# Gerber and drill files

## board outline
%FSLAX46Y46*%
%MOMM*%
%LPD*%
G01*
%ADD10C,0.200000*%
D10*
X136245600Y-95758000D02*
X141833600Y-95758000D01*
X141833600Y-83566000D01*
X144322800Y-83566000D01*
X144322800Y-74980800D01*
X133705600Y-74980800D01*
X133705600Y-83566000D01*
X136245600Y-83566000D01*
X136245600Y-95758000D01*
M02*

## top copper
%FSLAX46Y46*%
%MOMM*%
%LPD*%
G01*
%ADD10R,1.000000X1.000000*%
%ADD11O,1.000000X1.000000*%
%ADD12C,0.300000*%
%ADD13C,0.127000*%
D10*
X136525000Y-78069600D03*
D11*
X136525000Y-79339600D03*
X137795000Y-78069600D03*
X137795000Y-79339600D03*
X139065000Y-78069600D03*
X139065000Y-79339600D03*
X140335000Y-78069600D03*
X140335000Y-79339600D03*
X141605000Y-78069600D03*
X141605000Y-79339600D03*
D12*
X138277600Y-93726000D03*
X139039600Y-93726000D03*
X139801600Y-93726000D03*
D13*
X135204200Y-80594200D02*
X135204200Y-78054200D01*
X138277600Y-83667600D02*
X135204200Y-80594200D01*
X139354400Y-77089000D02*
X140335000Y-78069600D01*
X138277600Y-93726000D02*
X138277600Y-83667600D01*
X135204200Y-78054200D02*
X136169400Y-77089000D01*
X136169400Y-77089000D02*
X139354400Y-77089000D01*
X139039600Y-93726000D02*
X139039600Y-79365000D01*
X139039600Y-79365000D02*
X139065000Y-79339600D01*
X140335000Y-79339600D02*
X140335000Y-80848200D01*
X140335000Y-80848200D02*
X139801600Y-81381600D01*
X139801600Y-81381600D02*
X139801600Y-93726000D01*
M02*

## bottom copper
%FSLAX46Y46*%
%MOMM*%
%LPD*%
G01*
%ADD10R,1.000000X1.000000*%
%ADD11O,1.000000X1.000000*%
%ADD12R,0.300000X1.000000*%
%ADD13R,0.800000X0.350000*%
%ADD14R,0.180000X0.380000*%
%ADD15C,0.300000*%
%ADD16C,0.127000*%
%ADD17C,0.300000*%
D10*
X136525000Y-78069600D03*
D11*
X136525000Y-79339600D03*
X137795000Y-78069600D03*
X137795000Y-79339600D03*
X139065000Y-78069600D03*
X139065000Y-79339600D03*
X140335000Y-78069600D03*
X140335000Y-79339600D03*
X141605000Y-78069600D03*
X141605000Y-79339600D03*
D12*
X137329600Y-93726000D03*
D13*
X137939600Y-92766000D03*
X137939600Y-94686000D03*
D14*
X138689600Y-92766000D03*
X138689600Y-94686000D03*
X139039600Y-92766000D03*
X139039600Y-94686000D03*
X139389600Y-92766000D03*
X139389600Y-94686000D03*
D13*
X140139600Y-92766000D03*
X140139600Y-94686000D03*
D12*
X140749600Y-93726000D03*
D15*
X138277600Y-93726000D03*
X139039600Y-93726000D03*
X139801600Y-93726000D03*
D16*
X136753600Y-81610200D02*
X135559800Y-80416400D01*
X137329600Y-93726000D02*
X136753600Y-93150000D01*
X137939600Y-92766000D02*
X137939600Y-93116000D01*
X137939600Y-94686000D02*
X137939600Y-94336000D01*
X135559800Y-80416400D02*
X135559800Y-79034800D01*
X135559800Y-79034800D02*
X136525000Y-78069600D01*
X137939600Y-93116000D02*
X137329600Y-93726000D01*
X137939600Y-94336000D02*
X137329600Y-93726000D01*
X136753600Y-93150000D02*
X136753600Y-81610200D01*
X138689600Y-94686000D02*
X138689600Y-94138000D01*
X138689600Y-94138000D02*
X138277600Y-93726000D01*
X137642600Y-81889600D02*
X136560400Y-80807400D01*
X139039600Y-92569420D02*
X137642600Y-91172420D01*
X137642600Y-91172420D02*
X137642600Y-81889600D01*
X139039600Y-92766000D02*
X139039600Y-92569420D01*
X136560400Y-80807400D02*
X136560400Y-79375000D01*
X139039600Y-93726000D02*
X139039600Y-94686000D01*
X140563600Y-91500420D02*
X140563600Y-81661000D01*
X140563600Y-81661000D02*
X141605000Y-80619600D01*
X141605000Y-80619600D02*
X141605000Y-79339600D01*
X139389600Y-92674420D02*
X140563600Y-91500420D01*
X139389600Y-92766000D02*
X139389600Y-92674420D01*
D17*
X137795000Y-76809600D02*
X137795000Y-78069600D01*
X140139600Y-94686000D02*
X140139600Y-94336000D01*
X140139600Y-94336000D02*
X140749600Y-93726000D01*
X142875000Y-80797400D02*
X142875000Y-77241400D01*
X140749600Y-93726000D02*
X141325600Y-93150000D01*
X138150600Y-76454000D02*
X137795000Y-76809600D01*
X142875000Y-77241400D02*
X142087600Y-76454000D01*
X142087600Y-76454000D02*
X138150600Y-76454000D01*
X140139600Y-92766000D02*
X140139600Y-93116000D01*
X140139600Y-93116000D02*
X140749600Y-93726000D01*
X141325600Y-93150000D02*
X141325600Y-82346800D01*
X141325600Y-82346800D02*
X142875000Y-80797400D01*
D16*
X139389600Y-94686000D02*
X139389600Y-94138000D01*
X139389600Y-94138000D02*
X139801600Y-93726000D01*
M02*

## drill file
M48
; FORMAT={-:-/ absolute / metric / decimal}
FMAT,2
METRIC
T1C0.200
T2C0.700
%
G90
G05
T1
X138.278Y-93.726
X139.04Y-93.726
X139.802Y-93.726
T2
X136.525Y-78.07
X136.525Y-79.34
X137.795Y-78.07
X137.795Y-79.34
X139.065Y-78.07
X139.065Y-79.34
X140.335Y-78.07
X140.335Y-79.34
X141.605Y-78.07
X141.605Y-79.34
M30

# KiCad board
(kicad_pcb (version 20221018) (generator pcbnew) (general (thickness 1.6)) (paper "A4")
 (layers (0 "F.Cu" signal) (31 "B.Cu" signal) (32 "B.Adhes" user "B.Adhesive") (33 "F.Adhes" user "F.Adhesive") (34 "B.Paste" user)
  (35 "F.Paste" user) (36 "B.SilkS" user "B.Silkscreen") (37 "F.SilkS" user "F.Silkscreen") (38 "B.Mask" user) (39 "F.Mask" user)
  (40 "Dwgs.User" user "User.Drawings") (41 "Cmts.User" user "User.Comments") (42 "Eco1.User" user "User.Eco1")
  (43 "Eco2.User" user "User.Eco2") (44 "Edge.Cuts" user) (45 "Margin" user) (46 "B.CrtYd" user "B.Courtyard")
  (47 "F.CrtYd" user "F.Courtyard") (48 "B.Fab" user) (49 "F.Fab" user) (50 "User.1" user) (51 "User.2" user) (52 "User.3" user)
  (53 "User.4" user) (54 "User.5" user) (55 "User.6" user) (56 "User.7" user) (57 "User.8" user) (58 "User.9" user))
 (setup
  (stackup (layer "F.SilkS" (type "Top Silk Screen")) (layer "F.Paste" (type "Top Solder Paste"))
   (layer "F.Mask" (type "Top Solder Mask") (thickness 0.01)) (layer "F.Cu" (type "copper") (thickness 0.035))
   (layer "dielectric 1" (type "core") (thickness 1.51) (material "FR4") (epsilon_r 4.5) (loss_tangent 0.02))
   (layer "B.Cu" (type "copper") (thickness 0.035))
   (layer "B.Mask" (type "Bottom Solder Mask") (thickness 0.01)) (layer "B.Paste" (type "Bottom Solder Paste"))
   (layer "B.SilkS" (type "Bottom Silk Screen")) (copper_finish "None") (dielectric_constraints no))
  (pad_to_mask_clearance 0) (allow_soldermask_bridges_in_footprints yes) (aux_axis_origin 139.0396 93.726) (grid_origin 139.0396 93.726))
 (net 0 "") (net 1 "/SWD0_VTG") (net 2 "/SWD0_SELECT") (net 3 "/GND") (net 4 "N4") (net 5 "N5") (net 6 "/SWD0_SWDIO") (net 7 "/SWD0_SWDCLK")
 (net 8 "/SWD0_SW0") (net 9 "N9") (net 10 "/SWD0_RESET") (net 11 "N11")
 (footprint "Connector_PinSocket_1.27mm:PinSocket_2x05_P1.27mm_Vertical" (layer "F.Cu") (at 136.525 78.0696 90)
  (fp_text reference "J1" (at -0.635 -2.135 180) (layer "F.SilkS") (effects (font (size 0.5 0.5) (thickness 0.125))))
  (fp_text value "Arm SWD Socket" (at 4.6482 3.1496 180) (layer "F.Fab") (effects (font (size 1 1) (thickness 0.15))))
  (pad "1" thru_hole rect (at 0 0 90) (size 1 1) (drill 0.7) (layers "*.Cu" "*.Mask") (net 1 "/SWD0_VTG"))
  (pad "2" thru_hole oval (at -1.27 0 90) (size 1 1) (drill 0.7) (layers "*.Cu" "*.Mask") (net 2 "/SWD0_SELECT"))
  (pad "3" thru_hole oval (at 0 1.27 90) (size 1 1) (drill 0.7) (layers "*.Cu" "*.Mask") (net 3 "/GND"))
  (pad "4" thru_hole oval (at -1.27 1.27 90) (size 1 1) (drill 0.7) (layers "*.Cu" "*.Mask") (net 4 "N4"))
  (pad "5" thru_hole oval (at 0 2.54 90) (size 1 1) (drill 0.7) (layers "*.Cu" "*.Mask") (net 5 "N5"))
  (pad "6" thru_hole oval (at -1.27 2.54 90) (size 1 1) (drill 0.7) (layers "*.Cu" "*.Mask") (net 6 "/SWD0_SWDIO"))
  (pad "7" thru_hole oval (at 0 3.81 90) (size 1 1) (drill 0.7) (layers "*.Cu" "*.Mask") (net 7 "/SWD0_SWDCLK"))
  (pad "8" thru_hole oval (at -1.27 3.81 90) (size 1 1) (drill 0.7) (layers "*.Cu" "*.Mask") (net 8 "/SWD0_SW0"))
  (pad "9" thru_hole oval (at 0 5.08 90) (size 1 1) (drill 0.7) (layers "*.Cu" "*.Mask") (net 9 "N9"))
  (pad "10" thru_hole oval (at -1.27 5.08 90) (size 1 1) (drill 0.7) (layers "*.Cu" "*.Mask") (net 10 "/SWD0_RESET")))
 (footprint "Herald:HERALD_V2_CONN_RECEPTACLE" (layer "B.Cu") (at 139.0396 93.726)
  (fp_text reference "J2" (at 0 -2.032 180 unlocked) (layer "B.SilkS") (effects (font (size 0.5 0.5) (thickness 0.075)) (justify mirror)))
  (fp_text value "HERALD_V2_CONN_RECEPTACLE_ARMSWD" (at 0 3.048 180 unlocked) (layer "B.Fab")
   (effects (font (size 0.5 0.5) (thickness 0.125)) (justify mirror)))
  (pad "1" smd rect (at -1.71 0) (size 0.3 1) (layers "B.Cu" "B.Paste" "B.Mask") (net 1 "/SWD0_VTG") (thermal_bridge_angle 45))
  (pad "1" smd rect (at -1.1 -0.96) (size 0.8 0.35) (layers "B.Cu" "B.Paste" "B.Mask") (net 1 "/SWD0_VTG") (thermal_bridge_angle 45))
  (pad "1" smd rect (at -1.1 0.96) (size 0.8 0.35) (layers "B.Cu" "B.Paste" "B.Mask") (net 1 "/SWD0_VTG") (thermal_bridge_angle 45))
  (pad "2" smd rect (at -0.35 -0.96) (size 0.18 0.38) (layers "B.Cu" "B.Paste" "B.Mask") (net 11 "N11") (thermal_bridge_angle 45))
  (pad "3" smd rect (at -0.35 0.96) (size 0.18 0.38) (layers "B.Cu" "B.Paste" "B.Mask") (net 7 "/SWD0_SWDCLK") (thermal_bridge_angle 45))
  (pad "4" smd rect (at 0 -0.96) (size 0.18 0.38) (layers "B.Cu" "B.Paste" "B.Mask") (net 2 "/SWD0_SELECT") (thermal_bridge_angle 45))
  (pad "5" smd rect (at 0 0.96) (size 0.18 0.38) (layers "B.Cu" "B.Paste" "B.Mask") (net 6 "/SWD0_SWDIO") (thermal_bridge_angle 45))
  (pad "6" smd rect (at 0.35 -0.96) (size 0.18 0.38) (layers "B.Cu" "B.Paste" "B.Mask") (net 10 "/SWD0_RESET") (thermal_bridge_angle 45))
  (pad "7" smd rect (at 0.35 0.96) (size 0.18 0.38) (layers "B.Cu" "B.Paste" "B.Mask") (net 8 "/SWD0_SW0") (thermal_bridge_angle 45))
  (pad "8" smd rect (at 1.1 -0.96) (size 0.8 0.35) (layers "B.Cu" "B.Paste" "B.Mask") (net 3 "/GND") (thermal_bridge_angle 45))
  (pad "8" smd rect (at 1.1 0.96) (size 0.8 0.35) (layers "B.Cu" "B.Paste" "B.Mask") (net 3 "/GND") (thermal_bridge_angle 45))
  (pad "8" smd rect (at 1.71 0) (size 0.3 1) (layers "B.Cu" "B.Paste" "B.Mask") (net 3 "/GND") (thermal_bridge_angle 45)))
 (gr_poly
  (pts (xy 136.2456 95.758) (xy 141.8336 95.758) (xy 141.8336 83.566) (xy 144.3228 83.566) (xy 144.3228 74.9808) (xy 133.7056 74.9808)
   (xy 133.7056 83.566) (xy 136.2456 83.566))
  (stroke (width 0.2) (type solid)) (fill none) (layer "Edge.Cuts"))
 (segment (start 136.7536 81.6102) (end 135.5598 80.4164) (width 0.127) (layer "B.Cu") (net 1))
 (segment (start 137.3296 93.726) (end 136.7536 93.15) (width 0.127) (layer "B.Cu") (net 1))
 (segment (start 137.9396 92.766) (end 137.9396 93.116) (width 0.127) (layer "B.Cu") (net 1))
 (segment (start 137.9396 94.686) (end 137.9396 94.336) (width 0.127) (layer "B.Cu") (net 1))
 (segment (start 135.5598 80.4164) (end 135.5598 79.0348) (width 0.127) (layer "B.Cu") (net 1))
 (segment (start 135.5598 79.0348) (end 136.525 78.0696) (width 0.127) (layer "B.Cu") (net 1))
 (segment (start 137.9396 93.116) (end 137.3296 93.726) (width 0.127) (layer "B.Cu") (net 1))
 (segment (start 137.9396 94.336) (end 137.3296 93.726) (width 0.127) (layer "B.Cu") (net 1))
 (segment (start 136.7536 93.15) (end 136.7536 81.6102) (width 0.127) (layer "B.Cu") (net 1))
 (segment (start 135.2042 80.5942) (end 135.2042 78.0542) (width 0.127) (layer "F.Cu") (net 7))
 (segment (start 138.2776 83.6676) (end 135.2042 80.5942) (width 0.127) (layer "F.Cu") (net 7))
 (segment (start 139.3544 77.089) (end 140.335 78.0696) (width 0.127) (layer "F.Cu") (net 7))
 (segment (start 138.2776 93.726) (end 138.2776 83.6676) (width 0.127) (layer "F.Cu") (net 7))
 (segment (start 135.2042 78.0542) (end 136.1694 77.089) (width 0.127) (layer "F.Cu") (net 7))
 (segment (start 136.1694 77.089) (end 139.3544 77.089) (width 0.127) (layer "F.Cu") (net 7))
 (via (at 138.2776 93.726) (size 0.3) (drill 0.2) (layers "F.Cu" "B.Cu") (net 7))
 (segment (start 138.6896 94.686) (end 138.6896 94.138) (width 0.127) (layer "B.Cu") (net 7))
 (segment (start 138.6896 94.138) (end 138.2776 93.726) (width 0.127) (layer "B.Cu") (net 7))
 (segment (start 137.6426 81.8896) (end 136.5604 80.8074) (width 0.127) (layer "B.Cu") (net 2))
 (segment (start 139.0396 92.56942) (end 137.6426 91.17242) (width 0.127) (layer "B.Cu") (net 2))
 (segment (start 137.6426 91.17242) (end 137.6426 81.8896) (width 0.127) (layer "B.Cu") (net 2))
 (segment (start 139.0396 92.766) (end 139.0396 92.56942) (width 0.127) (layer "B.Cu") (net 2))
 (segment (start 136.5604 80.8074) (end 136.5604 79.375) (width 0.127) (layer "B.Cu") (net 2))
 (segment (start 139.0396 93.726) (end 139.0396 79.365) (width 0.127) (layer "F.Cu") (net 6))
 (segment (start 139.0396 79.365) (end 139.065 79.3396) (width 0.127) (layer "F.Cu") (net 6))
 (via (at 139.0396 93.726) (size 0.3) (drill 0.2) (layers "F.Cu" "B.Cu") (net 6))
 (segment (start 139.0396 93.726) (end 139.0396 94.686) (width 0.127) (layer "B.Cu") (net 6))
 (segment (start 140.5636 91.50042) (end 140.5636 81.661) (width 0.127) (layer "B.Cu") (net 10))
 (segment (start 140.5636 81.661) (end 141.605 80.6196) (width 0.127) (layer "B.Cu") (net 10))
 (segment (start 141.605 80.6196) (end 141.605 79.3396) (width 0.127) (layer "B.Cu") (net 10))
 (segment (start 139.3896 92.67442) (end 140.5636 91.50042) (width 0.127) (layer "B.Cu") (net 10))
 (segment (start 139.3896 92.766) (end 139.3896 92.67442) (width 0.127) (layer "B.Cu") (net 10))
 (segment (start 137.795 76.8096) (end 137.795 78.0696) (width 0.3) (layer "B.Cu") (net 3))
 (segment (start 140.1396 94.686) (end 140.1396 94.336) (width 0.3) (layer "B.Cu") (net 3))
 (segment (start 140.1396 94.336) (end 140.7496 93.726) (width 0.3) (layer "B.Cu") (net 3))
 (segment (start 142.875 80.7974) (end 142.875 77.2414) (width 0.3) (layer "B.Cu") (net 3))
 (segment (start 140.7496 93.726) (end 141.3256 93.15) (width 0.3) (layer "B.Cu") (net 3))
 (segment (start 138.1506 76.454) (end 137.795 76.8096) (width 0.3) (layer "B.Cu") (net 3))
 (segment (start 142.875 77.2414) (end 142.0876 76.454) (width 0.3) (layer "B.Cu") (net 3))
 (segment (start 142.0876 76.454) (end 138.1506 76.454) (width 0.3) (layer "B.Cu") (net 3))
 (segment (start 140.1396 92.766) (end 140.1396 93.116) (width 0.3) (layer "B.Cu") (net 3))
 (segment (start 140.1396 93.116) (end 140.7496 93.726) (width 0.3) (layer "B.Cu") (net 3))
 (segment (start 141.3256 93.15) (end 141.3256 82.3468) (width 0.3) (layer "B.Cu") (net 3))
 (segment (start 141.3256 82.3468) (end 142.875 80.7974) (width 0.3) (layer "B.Cu") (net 3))
 (segment (start 140.335 79.3396) (end 140.335 80.8482) (width 0.127) (layer "F.Cu") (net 8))
 (segment (start 140.335 80.8482) (end 139.8016 81.3816) (width 0.127) (layer "F.Cu") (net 8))
 (segment (start 139.8016 81.3816) (end 139.8016 93.726) (width 0.127) (layer "F.Cu") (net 8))
 (via (at 139.8016 93.726) (size 0.3) (drill 0.2) (layers "F.Cu" "B.Cu") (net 8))
 (segment (start 139.3896 94.686) (end 139.3896 94.138) (width 0.127) (layer "B.Cu") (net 8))
 (segment (start 139.3896 94.138) (end 139.8016 93.726) (width 0.127) (layer "B.Cu") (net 8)))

